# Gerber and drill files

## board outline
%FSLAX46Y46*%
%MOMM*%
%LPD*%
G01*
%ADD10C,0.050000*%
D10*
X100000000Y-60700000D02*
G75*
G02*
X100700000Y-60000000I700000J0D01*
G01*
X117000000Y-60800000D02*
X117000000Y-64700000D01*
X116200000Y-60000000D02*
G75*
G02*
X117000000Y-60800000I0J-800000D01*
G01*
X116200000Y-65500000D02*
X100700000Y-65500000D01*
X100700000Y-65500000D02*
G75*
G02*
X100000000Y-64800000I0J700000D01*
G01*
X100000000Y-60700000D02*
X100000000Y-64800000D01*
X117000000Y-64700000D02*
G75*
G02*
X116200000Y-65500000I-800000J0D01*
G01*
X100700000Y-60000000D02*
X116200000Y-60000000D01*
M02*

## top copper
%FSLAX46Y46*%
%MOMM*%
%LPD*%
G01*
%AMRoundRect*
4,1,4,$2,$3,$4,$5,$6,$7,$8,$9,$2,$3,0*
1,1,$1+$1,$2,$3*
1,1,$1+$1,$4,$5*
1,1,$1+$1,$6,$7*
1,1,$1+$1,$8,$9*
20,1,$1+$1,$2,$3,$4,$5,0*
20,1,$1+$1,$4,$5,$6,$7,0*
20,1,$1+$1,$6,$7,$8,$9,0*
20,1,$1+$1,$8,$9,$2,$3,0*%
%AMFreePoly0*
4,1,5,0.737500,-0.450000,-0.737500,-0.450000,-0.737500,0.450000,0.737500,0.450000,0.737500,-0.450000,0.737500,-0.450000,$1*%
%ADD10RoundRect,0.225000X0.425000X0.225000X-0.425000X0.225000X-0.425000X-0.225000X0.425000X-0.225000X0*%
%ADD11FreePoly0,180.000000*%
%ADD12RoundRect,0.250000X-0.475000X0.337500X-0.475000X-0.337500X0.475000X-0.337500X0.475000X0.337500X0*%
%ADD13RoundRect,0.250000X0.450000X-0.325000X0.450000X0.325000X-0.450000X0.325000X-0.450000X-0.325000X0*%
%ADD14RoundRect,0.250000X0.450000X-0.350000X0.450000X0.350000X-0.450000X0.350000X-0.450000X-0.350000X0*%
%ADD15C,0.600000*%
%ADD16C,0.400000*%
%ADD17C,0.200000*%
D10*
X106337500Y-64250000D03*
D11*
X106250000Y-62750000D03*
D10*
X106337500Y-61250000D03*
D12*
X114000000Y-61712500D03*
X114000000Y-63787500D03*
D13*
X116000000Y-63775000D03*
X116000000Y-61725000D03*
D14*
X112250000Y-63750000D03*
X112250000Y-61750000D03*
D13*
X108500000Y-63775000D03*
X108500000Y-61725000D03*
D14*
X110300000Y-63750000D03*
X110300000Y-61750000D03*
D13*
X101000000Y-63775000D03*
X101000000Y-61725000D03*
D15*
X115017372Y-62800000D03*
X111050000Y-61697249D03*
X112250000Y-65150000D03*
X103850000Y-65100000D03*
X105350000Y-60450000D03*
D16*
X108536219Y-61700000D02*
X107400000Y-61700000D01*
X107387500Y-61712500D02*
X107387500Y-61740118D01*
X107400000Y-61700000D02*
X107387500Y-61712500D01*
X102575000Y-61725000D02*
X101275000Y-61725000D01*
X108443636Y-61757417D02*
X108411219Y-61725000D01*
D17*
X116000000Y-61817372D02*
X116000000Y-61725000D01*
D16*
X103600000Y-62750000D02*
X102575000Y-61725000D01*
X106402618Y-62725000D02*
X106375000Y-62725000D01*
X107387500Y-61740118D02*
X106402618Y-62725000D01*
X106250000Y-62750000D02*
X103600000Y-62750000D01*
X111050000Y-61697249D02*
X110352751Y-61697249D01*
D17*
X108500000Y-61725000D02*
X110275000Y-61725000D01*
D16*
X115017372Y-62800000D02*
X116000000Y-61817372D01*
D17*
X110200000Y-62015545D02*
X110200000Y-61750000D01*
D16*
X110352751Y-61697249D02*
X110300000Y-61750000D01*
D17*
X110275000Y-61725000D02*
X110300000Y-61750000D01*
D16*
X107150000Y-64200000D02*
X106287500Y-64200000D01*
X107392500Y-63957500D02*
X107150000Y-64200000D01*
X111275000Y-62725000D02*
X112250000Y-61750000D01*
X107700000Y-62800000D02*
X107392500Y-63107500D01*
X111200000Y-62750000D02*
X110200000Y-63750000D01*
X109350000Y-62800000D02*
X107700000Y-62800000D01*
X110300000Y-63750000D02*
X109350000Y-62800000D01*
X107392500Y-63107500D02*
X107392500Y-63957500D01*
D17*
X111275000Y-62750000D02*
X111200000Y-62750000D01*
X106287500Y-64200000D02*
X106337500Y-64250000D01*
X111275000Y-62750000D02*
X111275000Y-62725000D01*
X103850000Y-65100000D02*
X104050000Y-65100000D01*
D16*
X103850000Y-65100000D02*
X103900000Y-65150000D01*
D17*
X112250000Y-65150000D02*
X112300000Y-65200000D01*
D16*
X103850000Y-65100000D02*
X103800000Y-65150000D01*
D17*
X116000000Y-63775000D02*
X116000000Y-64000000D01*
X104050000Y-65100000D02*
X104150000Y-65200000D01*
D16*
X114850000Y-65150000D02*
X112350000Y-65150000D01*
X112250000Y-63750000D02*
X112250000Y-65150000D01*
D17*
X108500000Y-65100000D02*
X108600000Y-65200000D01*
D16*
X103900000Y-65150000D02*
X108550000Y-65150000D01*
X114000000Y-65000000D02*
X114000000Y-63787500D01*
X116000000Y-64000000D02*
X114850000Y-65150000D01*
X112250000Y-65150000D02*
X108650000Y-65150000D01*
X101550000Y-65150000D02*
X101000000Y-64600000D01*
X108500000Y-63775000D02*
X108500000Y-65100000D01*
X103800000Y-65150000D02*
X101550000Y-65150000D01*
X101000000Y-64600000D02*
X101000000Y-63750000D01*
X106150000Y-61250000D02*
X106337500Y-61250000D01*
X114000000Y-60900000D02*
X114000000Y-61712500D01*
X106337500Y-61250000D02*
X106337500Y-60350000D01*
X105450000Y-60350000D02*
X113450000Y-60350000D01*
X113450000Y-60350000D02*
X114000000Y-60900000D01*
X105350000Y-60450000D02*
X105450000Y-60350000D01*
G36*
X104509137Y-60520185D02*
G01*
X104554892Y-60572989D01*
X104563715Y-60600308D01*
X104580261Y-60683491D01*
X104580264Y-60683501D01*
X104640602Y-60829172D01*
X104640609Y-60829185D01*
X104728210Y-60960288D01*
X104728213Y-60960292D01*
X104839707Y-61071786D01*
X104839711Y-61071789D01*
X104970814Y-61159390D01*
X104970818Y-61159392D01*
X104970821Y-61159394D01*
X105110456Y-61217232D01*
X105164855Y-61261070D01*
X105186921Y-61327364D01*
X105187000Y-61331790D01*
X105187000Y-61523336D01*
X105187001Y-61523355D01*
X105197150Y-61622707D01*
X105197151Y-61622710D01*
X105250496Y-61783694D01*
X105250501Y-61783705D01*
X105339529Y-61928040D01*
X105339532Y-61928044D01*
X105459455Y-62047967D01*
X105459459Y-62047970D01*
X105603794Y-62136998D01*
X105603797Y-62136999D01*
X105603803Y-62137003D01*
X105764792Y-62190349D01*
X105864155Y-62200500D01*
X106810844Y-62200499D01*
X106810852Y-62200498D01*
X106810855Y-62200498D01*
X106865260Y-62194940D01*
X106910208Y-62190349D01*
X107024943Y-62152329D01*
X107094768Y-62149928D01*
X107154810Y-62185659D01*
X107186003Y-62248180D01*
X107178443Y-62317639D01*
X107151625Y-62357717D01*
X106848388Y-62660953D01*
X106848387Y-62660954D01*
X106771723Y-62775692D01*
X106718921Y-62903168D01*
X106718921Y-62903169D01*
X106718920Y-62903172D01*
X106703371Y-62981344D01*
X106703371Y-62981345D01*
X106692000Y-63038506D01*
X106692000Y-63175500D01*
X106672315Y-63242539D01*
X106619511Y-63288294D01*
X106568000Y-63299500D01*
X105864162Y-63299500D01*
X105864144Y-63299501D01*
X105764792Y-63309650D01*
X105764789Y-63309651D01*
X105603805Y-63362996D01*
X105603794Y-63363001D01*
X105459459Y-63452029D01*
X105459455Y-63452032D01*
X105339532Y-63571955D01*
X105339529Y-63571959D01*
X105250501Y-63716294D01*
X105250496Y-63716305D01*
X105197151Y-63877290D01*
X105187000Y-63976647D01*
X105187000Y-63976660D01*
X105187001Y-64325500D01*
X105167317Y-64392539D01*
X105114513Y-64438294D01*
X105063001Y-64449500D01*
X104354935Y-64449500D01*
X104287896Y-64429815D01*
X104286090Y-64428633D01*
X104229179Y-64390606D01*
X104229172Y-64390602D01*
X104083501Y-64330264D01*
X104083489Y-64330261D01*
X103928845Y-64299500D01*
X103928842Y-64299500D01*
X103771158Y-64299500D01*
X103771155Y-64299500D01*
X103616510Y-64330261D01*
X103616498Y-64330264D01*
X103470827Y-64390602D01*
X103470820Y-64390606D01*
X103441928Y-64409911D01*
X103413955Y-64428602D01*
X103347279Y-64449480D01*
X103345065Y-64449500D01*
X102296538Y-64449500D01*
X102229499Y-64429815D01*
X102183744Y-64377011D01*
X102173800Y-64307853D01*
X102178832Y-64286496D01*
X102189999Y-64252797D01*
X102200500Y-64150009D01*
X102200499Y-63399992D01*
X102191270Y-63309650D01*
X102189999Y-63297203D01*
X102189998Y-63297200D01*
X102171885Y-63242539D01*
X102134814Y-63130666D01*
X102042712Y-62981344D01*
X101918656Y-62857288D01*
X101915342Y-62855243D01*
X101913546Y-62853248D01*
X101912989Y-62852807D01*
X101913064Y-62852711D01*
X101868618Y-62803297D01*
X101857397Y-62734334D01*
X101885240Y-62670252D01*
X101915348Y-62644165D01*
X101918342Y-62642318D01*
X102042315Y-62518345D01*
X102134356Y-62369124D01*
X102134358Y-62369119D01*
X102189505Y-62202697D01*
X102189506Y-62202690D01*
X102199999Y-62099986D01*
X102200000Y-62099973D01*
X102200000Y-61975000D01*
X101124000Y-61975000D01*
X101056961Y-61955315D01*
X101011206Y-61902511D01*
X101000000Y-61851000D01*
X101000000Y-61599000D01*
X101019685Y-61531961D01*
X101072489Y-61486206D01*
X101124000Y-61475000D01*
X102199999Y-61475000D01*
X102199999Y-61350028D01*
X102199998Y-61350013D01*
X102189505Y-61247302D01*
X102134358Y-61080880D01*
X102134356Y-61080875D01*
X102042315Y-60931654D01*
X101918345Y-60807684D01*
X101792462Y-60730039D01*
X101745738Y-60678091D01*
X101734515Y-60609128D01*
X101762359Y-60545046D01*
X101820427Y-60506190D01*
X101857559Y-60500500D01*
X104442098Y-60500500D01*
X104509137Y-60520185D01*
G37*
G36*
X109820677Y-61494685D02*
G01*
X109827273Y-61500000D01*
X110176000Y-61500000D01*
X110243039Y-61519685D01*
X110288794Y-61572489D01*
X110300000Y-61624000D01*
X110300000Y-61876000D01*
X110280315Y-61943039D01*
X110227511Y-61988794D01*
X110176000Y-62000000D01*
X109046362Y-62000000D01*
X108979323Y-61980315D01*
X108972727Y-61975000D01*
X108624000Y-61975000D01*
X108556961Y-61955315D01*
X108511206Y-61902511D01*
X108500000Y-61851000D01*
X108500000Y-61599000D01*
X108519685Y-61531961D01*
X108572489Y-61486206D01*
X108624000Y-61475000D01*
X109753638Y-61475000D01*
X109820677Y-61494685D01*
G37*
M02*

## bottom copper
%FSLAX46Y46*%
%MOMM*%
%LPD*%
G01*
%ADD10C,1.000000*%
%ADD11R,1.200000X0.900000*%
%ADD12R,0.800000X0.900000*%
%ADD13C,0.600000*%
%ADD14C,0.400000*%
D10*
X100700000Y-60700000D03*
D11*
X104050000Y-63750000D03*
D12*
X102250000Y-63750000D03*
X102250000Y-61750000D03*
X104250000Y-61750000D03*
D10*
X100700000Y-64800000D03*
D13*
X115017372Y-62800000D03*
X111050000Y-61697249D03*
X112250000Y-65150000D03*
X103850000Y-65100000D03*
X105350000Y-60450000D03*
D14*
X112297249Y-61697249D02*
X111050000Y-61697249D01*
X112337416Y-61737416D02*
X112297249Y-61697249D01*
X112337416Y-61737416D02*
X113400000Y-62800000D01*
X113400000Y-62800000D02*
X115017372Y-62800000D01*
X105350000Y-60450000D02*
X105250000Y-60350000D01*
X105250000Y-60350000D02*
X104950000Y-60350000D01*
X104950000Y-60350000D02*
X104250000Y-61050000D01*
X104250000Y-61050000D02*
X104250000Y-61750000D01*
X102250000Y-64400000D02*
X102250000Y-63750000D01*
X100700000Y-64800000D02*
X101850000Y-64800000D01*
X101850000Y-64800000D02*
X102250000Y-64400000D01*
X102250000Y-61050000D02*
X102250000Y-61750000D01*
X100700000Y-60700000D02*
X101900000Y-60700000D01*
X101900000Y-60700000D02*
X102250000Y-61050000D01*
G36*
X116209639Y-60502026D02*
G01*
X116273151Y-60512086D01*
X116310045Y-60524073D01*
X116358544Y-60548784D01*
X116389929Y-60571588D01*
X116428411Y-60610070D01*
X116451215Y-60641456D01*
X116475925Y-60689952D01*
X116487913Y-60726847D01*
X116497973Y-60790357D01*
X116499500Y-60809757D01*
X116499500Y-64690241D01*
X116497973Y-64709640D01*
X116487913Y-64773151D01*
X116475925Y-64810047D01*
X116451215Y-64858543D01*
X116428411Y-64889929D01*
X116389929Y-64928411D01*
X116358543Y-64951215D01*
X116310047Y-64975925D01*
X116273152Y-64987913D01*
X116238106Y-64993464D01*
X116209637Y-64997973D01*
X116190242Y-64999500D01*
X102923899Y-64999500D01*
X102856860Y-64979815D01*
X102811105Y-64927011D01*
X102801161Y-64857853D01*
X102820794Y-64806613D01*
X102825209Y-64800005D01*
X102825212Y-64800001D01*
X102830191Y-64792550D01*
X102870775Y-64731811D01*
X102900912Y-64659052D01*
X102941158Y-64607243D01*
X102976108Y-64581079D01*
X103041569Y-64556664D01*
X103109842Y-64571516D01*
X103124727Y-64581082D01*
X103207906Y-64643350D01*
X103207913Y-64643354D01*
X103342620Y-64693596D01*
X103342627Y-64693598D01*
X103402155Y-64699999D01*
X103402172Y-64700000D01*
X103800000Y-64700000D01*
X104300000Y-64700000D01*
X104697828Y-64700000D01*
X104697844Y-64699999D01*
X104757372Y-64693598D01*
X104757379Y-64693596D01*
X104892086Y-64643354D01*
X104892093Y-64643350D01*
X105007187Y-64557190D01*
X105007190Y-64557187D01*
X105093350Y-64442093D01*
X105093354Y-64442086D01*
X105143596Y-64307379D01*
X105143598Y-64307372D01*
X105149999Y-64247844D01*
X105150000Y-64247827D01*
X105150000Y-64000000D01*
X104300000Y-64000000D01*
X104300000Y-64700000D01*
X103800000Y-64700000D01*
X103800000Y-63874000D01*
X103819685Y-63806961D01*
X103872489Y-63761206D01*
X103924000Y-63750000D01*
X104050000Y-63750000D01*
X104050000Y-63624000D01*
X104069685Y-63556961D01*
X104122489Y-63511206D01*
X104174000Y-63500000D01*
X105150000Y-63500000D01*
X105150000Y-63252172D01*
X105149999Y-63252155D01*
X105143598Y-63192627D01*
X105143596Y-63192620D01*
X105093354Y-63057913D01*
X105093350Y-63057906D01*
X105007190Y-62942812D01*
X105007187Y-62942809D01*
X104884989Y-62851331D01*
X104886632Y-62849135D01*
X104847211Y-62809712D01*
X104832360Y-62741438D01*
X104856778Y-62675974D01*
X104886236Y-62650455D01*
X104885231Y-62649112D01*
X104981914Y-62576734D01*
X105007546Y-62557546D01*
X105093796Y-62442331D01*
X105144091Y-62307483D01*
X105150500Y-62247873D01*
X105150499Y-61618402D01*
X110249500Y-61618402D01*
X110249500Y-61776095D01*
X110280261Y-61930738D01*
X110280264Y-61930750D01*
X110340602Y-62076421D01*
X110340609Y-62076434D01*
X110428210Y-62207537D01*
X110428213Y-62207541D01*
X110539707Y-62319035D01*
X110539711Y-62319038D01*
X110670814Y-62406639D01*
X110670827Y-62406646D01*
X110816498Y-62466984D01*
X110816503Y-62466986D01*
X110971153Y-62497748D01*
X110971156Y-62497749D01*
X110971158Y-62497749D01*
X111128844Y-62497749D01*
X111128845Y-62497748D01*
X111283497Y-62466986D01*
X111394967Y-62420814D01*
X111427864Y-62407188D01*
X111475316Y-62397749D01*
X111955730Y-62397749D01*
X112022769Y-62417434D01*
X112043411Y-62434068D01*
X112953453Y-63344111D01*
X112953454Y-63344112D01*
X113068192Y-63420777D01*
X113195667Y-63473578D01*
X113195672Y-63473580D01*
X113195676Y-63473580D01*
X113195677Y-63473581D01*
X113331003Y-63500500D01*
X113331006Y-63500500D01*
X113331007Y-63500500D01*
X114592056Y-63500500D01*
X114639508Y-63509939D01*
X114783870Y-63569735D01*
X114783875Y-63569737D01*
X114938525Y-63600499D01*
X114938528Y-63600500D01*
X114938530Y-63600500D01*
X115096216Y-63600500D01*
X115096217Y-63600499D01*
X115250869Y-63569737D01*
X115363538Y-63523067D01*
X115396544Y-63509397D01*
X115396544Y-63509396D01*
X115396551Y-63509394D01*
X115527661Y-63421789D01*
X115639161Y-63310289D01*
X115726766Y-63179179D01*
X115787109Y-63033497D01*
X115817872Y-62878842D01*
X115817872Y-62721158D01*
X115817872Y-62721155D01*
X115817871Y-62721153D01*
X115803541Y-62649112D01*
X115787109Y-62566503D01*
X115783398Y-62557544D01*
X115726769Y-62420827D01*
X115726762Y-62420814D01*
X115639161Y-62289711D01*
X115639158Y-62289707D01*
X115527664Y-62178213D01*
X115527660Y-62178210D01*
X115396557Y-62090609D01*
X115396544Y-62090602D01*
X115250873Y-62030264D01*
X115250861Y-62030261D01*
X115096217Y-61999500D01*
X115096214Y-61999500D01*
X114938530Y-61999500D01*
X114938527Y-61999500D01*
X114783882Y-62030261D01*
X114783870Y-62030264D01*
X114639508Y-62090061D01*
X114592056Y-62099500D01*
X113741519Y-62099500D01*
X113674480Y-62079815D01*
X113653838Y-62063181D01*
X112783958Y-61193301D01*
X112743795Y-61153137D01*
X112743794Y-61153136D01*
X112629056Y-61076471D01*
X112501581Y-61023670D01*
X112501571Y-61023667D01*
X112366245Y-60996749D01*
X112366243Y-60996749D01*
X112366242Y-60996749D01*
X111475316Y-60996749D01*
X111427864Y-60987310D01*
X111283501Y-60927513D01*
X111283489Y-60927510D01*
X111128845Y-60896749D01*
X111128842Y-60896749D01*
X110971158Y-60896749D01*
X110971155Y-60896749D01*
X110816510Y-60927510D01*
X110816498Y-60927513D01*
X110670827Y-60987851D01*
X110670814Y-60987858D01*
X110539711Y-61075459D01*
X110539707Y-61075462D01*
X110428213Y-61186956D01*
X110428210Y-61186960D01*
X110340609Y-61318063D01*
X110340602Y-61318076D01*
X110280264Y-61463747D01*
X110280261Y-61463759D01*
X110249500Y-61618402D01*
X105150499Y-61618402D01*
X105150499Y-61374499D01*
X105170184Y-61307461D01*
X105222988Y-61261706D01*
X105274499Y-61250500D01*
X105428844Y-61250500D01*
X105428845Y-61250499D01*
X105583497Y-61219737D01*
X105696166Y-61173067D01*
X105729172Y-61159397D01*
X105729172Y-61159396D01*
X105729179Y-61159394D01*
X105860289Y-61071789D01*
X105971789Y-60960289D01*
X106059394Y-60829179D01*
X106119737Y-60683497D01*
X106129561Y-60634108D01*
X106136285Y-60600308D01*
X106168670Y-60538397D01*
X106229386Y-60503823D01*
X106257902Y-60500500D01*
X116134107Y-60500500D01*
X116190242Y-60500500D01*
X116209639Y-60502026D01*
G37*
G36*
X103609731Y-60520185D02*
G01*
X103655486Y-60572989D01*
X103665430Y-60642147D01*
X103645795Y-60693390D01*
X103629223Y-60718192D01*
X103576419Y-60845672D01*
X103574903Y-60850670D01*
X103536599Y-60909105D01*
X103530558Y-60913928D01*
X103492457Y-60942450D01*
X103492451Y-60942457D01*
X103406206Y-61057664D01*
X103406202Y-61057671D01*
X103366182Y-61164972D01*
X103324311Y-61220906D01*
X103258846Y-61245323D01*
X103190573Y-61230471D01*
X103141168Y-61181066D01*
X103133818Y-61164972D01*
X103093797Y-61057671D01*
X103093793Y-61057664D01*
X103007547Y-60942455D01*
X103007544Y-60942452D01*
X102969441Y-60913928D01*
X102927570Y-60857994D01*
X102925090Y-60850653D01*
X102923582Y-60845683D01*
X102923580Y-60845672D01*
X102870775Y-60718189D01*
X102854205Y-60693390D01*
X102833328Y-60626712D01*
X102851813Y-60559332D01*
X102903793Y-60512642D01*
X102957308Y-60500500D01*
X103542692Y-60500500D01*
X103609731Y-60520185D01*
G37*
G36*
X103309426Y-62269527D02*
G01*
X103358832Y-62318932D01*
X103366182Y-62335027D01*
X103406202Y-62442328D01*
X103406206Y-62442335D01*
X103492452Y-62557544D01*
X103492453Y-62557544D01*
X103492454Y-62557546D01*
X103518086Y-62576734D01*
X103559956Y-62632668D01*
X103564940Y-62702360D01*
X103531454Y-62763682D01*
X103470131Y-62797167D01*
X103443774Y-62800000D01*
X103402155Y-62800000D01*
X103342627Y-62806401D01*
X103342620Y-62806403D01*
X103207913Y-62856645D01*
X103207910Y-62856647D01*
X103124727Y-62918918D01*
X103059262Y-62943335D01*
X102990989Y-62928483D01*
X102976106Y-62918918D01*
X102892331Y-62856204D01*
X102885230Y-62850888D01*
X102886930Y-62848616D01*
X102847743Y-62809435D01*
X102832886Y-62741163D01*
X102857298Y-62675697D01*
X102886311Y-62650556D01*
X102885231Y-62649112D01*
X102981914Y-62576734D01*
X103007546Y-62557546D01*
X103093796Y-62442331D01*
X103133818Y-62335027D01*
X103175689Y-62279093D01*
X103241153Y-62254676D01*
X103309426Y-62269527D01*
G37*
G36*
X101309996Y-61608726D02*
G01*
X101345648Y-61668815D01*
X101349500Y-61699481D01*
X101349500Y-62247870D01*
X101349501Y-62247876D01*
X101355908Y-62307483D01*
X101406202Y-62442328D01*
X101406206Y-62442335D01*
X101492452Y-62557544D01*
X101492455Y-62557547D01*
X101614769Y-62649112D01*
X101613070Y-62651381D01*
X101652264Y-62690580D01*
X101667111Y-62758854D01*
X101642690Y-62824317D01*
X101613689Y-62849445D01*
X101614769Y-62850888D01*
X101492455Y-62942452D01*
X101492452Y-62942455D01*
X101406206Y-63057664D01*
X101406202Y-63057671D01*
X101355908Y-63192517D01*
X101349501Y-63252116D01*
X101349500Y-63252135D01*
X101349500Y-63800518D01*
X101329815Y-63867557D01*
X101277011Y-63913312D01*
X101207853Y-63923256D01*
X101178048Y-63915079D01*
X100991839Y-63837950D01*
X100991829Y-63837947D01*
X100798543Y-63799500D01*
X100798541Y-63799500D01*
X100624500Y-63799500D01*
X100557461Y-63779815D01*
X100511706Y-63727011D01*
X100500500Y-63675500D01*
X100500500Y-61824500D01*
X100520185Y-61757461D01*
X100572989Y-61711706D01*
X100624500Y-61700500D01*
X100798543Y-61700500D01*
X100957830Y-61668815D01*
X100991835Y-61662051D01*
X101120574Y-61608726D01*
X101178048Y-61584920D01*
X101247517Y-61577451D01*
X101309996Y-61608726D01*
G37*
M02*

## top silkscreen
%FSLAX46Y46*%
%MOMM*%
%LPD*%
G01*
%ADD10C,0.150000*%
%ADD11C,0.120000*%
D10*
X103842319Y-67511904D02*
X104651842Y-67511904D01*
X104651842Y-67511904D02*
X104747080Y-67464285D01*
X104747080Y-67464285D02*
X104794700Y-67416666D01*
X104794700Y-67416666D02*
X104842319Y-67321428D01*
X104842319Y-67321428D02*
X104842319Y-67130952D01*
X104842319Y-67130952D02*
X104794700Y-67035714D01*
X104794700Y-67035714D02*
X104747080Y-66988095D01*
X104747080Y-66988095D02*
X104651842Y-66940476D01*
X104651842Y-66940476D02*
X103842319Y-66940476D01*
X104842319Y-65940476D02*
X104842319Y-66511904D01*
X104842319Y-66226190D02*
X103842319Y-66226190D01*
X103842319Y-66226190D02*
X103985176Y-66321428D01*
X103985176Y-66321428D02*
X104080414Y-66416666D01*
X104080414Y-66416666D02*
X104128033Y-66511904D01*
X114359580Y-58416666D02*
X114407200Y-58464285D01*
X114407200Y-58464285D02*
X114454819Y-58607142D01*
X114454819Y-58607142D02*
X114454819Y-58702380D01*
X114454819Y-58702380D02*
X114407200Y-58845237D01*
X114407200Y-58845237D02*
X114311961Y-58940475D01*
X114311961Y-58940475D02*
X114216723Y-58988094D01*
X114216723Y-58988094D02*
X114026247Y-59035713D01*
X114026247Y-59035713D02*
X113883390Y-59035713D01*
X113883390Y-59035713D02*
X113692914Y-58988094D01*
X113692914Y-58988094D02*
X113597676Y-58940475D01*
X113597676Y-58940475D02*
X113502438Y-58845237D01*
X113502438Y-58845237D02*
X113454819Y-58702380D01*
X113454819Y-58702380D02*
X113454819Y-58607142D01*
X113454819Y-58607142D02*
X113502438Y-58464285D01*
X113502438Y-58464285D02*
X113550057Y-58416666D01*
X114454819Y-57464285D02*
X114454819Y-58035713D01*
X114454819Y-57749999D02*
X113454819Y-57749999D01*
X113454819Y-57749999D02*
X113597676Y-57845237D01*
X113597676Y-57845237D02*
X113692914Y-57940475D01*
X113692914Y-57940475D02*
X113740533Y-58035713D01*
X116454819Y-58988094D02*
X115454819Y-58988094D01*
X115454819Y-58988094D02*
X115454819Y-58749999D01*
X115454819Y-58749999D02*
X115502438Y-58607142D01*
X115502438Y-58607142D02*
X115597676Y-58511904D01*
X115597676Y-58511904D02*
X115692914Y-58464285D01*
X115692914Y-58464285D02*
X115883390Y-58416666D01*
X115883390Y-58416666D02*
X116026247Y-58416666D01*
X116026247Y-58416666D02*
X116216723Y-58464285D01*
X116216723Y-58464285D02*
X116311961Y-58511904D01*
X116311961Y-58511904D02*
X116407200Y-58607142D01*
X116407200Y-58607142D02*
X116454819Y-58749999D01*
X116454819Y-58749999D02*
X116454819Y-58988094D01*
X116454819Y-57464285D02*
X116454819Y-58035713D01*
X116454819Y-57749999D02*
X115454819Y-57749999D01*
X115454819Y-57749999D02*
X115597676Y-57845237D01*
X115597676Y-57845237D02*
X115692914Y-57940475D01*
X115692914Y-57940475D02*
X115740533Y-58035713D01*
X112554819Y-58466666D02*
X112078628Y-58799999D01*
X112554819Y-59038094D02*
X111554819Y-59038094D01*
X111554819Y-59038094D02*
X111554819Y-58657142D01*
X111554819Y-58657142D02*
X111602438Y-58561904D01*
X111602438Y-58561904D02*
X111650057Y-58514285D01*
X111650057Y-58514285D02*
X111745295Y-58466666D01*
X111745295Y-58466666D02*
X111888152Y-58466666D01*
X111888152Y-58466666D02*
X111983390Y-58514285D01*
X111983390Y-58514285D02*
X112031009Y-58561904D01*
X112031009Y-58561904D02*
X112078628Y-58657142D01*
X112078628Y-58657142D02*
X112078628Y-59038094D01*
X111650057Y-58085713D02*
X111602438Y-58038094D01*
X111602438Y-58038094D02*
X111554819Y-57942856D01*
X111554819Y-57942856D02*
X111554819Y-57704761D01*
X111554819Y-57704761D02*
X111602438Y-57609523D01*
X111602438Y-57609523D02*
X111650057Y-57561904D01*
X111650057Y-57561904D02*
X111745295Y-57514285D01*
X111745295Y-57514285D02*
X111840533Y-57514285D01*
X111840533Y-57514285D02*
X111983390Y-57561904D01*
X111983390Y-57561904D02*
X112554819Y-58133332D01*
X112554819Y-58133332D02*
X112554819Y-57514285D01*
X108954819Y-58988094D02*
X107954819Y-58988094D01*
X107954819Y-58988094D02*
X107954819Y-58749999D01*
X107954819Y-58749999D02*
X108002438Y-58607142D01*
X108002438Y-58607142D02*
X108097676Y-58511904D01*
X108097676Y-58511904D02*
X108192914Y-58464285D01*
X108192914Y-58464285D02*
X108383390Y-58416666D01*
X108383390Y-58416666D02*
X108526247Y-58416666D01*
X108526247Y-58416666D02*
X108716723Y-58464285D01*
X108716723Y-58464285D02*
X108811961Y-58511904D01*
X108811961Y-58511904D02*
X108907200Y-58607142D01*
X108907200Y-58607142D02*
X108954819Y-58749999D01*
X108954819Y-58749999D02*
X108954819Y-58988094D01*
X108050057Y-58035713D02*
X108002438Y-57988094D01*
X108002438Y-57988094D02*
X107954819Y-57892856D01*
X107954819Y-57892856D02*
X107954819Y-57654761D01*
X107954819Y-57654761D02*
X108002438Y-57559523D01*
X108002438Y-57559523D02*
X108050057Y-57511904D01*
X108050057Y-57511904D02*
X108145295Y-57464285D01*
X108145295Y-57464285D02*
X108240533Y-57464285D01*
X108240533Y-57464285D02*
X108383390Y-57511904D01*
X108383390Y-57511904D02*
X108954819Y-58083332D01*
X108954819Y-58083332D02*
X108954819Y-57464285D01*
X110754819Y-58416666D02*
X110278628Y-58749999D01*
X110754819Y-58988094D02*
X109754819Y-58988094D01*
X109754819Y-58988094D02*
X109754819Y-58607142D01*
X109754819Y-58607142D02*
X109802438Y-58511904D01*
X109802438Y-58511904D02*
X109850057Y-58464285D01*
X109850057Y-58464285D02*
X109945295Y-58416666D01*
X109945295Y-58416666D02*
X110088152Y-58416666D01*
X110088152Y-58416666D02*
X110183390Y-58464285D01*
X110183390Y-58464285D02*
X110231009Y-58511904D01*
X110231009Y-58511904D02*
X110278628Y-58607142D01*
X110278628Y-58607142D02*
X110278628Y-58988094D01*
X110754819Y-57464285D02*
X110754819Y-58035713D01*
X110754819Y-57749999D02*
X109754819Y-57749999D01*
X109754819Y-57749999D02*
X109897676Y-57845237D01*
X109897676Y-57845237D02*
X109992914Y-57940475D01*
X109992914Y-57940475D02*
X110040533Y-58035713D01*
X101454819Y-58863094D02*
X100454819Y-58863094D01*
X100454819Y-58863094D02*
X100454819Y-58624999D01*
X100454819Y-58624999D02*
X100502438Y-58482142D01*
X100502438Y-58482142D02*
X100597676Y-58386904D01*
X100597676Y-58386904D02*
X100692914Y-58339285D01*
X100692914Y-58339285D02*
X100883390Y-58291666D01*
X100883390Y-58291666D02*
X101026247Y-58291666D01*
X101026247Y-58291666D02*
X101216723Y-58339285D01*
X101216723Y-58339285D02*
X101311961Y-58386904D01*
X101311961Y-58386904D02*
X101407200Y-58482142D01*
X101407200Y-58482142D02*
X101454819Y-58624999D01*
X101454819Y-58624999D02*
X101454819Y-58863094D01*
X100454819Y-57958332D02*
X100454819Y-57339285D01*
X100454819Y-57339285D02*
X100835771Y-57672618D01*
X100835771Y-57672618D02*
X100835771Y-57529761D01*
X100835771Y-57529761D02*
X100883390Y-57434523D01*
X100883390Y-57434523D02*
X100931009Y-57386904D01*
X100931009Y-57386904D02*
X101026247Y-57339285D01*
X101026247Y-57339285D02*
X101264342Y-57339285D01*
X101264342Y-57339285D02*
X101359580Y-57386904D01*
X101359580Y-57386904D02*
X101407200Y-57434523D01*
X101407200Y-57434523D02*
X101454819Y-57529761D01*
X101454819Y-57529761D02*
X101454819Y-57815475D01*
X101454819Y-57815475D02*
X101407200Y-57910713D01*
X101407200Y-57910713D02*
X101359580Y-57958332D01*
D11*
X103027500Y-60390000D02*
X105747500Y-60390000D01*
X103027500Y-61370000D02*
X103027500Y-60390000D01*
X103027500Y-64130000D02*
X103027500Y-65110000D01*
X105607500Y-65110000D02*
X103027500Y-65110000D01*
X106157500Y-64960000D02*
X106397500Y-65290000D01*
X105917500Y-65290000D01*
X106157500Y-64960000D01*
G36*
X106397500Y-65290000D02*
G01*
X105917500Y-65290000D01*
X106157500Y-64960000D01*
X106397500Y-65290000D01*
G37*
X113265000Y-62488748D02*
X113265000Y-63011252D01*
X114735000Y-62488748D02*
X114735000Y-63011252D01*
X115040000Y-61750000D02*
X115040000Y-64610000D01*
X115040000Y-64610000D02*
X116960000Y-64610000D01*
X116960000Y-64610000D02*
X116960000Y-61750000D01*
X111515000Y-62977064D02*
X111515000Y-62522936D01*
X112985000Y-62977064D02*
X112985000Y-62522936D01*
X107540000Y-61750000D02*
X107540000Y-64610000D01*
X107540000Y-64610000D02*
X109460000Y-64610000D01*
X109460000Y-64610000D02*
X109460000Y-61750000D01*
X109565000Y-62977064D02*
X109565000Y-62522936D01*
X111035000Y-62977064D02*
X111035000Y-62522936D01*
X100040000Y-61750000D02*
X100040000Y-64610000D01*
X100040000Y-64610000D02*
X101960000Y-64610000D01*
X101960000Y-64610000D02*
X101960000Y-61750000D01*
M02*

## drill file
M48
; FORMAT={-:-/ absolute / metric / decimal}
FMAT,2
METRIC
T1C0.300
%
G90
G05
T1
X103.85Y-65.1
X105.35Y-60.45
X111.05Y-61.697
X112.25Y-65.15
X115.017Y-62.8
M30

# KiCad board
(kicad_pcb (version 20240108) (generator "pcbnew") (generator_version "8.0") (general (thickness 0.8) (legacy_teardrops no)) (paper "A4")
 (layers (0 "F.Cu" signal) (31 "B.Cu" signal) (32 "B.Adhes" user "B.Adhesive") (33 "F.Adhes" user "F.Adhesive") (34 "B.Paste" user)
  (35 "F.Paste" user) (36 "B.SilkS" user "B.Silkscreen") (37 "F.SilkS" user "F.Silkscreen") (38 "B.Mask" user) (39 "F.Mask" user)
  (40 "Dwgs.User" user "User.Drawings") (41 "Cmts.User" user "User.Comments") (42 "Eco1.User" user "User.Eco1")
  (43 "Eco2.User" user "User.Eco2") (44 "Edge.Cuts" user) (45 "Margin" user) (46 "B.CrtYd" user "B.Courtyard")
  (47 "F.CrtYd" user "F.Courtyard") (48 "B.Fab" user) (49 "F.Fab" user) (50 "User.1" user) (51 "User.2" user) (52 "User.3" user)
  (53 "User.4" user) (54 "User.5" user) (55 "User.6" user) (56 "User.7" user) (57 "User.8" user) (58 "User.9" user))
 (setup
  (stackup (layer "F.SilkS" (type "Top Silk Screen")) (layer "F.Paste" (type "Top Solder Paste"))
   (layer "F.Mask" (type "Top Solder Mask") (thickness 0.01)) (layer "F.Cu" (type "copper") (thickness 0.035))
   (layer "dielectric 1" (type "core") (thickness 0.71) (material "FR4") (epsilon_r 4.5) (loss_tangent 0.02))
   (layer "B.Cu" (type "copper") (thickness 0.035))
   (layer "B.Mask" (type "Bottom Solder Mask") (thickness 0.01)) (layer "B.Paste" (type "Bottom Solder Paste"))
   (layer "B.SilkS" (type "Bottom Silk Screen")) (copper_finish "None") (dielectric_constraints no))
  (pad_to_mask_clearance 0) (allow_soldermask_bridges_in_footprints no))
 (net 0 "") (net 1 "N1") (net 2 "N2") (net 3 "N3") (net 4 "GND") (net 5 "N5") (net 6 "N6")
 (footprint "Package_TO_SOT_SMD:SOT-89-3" (layer "F.Cu") (at 104.3875 62.75 180)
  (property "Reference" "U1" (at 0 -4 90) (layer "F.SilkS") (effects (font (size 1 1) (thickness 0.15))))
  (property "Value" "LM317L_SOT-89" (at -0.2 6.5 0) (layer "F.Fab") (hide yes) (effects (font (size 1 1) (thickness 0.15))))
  (fp_line (start 1.36 2.36) (end -1.36 2.36) (stroke (width 0.12) (type solid)) (layer "F.SilkS"))
  (fp_line (start 1.36 1.38) (end 1.36 2.36) (stroke (width 0.12) (type solid)) (layer "F.SilkS"))
  (fp_line (start 1.36 -1.38) (end 1.36 -2.36) (stroke (width 0.12) (type solid)) (layer "F.SilkS"))
  (fp_line (start -1.22 -2.36) (end 1.36 -2.36) (stroke (width 0.12) (type solid)) (layer "F.SilkS"))
  (fp_poly
   (pts (xy -1.77 -2.21) (xy -2.01 -2.54) (xy -1.53 -2.54) (xy -1.77 -2.21)) (stroke (width 0.12) (type solid)) (fill solid)
   (layer "F.SilkS"))
  (pad "1" smd roundrect (at -1.95 -1.5 180) (size 1.3 0.9) (layers "F.Cu" "F.Paste" "F.Mask") (roundrect_rratio 0.25) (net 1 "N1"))
  (pad "2" smd custom (at -1.8625 0 180) (size 1.475 0.9) (layers "F.Cu" "F.Paste" "F.Mask") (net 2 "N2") (zone_connect 2)
   (thermal_bridge_angle 45) (options (clearance outline) (anchor rect)) (primitives))
  (pad "3" smd roundrect (at -1.95 1.5 180) (size 1.3 0.9) (layers "F.Cu" "F.Paste" "F.Mask") (roundrect_rratio 0.25) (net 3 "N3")))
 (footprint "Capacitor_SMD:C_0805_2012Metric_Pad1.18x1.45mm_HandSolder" (layer "F.Cu") (at 114 62.75 -90)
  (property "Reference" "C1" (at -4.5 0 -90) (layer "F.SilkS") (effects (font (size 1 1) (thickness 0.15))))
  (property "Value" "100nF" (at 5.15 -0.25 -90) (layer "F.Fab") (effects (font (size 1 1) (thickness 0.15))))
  (fp_line (start -0.261252 0.735) (end 0.261252 0.735) (stroke (width 0.12) (type solid)) (layer "F.SilkS"))
  (fp_line (start -0.261252 -0.735) (end 0.261252 -0.735) (stroke (width 0.12) (type solid)) (layer "F.SilkS"))
  (pad "1" smd roundrect (at -1.0375 0 270) (size 1.175 1.45) (layers "F.Cu" "F.Paste" "F.Mask") (roundrect_rratio 0.212766) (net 3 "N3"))
  (pad "2" smd roundrect (at 1.0375 0 270) (size 1.175 1.45) (layers "F.Cu" "F.Paste" "F.Mask") (roundrect_rratio 0.212766) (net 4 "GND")))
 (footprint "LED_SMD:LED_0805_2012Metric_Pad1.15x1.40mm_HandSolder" (layer "F.Cu") (at 116 62.75 90)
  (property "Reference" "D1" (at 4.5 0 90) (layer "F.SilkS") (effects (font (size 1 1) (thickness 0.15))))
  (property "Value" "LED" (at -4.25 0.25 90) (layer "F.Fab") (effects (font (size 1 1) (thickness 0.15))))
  (fp_line (start 1 -0.96) (end -1.86 -0.96) (stroke (width 0.12) (type solid)) (layer "F.SilkS"))
  (fp_line (start -1.86 -0.96) (end -1.86 0.96) (stroke (width 0.12) (type solid)) (layer "F.SilkS"))
  (fp_line (start -1.86 0.96) (end 1 0.96) (stroke (width 0.12) (type solid)) (layer "F.SilkS"))
  (pad "1" smd roundrect (at -1.025 0 90) (size 1.15 1.4) (layers "F.Cu" "F.Paste" "F.Mask") (roundrect_rratio 0.217391) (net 4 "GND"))
  (pad "2" smd roundrect (at 1.025 0 90) (size 1.15 1.4) (layers "F.Cu" "F.Paste" "F.Mask") (roundrect_rratio 0.217391) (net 2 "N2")))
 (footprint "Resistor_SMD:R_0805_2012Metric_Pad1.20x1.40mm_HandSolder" (layer "F.Cu") (at 112.25 62.75 90)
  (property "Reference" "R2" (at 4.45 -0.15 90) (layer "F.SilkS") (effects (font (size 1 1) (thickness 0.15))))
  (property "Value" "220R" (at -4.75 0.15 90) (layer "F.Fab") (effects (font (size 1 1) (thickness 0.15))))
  (fp_line (start -0.227064 -0.735) (end 0.227064 -0.735) (stroke (width 0.12) (type solid)) (layer "F.SilkS"))
  (fp_line (start -0.227064 0.735) (end 0.227064 0.735) (stroke (width 0.12) (type solid)) (layer "F.SilkS"))
  (pad "1" smd roundrect (at -1 0 90) (size 1.2 1.4) (layers "F.Cu" "F.Paste" "F.Mask") (roundrect_rratio 0.208333) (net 4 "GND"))
  (pad "2" smd roundrect (at 1 0 90) (size 1.2 1.4) (layers "F.Cu" "F.Paste" "F.Mask") (roundrect_rratio 0.208333) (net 1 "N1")))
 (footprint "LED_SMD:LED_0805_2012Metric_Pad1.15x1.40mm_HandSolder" (layer "F.Cu") (at 108.5 62.75 90)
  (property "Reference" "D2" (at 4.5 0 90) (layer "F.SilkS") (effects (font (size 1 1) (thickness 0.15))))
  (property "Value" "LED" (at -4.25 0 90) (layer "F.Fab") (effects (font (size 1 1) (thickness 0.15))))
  (fp_line (start 1 -0.96) (end -1.86 -0.96) (stroke (width 0.12) (type solid)) (layer "F.SilkS"))
  (fp_line (start -1.86 -0.96) (end -1.86 0.96) (stroke (width 0.12) (type solid)) (layer "F.SilkS"))
  (fp_line (start -1.86 0.96) (end 1 0.96) (stroke (width 0.12) (type solid)) (layer "F.SilkS"))
  (pad "1" smd roundrect (at -1.025 0 90) (size 1.15 1.4) (layers "F.Cu" "F.Paste" "F.Mask") (roundrect_rratio 0.217391) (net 4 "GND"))
  (pad "2" smd roundrect (at 1.025 0 90) (size 1.15 1.4) (layers "F.Cu" "F.Paste" "F.Mask") (roundrect_rratio 0.217391) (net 2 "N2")))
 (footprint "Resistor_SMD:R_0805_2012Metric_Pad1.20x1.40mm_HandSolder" (layer "F.Cu") (at 110.3 62.75 90)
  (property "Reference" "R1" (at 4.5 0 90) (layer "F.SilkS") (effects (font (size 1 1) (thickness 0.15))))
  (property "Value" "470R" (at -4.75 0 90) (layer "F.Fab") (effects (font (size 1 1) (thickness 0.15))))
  (fp_line (start -0.227064 -0.735) (end 0.227064 -0.735) (stroke (width 0.12) (type solid)) (layer "F.SilkS"))
  (fp_line (start -0.227064 0.735) (end 0.227064 0.735) (stroke (width 0.12) (type solid)) (layer "F.SilkS"))
  (pad "1" smd roundrect (at -1 0 90) (size 1.2 1.4) (layers "F.Cu" "F.Paste" "F.Mask") (roundrect_rratio 0.208333) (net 1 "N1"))
  (pad "2" smd roundrect (at 1 0 90) (size 1.2 1.4) (layers "F.Cu" "F.Paste" "F.Mask") (roundrect_rratio 0.208333) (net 2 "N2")))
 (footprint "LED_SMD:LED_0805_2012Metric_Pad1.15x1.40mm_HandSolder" (layer "F.Cu") (at 101 62.75 90)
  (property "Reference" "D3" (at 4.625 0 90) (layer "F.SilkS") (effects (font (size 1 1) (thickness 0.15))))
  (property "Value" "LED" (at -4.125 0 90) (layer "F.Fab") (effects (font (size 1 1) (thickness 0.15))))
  (fp_line (start 1 -0.96) (end -1.86 -0.96) (stroke (width 0.12) (type solid)) (layer "F.SilkS"))
  (fp_line (start -1.86 -0.96) (end -1.86 0.96) (stroke (width 0.12) (type solid)) (layer "F.SilkS"))
  (fp_line (start -1.86 0.96) (end 1 0.96) (stroke (width 0.12) (type solid)) (layer "F.SilkS"))
  (pad "1" smd roundrect (at -1.025 0 90) (size 1.15 1.4) (layers "F.Cu" "F.Paste" "F.Mask") (roundrect_rratio 0.217391) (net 4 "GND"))
  (pad "2" smd roundrect (at 1.025 0 90) (size 1.15 1.4) (layers "F.Cu" "F.Paste" "F.Mask") (roundrect_rratio 0.217391) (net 2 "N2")))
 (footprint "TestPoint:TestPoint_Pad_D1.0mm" (layer "B.Cu") (at 100.7 60.7 180)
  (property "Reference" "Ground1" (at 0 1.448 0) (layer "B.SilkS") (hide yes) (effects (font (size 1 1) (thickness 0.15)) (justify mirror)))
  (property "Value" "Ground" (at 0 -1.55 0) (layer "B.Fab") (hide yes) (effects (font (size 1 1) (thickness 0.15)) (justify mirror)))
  (pad "1" smd circle (at 0 0 180) (size 1 1) (layers "B.Cu" "B.Mask") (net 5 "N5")))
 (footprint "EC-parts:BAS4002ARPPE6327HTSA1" (layer "B.Cu") (at 103.25 62.75 180)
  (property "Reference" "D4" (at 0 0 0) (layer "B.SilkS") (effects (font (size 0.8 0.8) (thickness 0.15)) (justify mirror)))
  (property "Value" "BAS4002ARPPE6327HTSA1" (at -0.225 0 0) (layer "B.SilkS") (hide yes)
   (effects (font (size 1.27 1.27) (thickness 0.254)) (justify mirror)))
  (pad "1" smd rect (at -0.8 -1 90) (size 0.9 1.2) (layers "B.Cu" "B.Paste" "B.Mask") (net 4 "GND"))
  (pad "2" smd rect (at 1 -1 180) (size 0.8 0.9) (layers "B.Cu" "B.Paste" "B.Mask") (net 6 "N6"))
  (pad "3" smd rect (at 1 1 180) (size 0.8 0.9) (layers "B.Cu" "B.Paste" "B.Mask") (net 5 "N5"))
  (pad "4" smd rect (at -1 1 180) (size 0.8 0.9) (layers "B.Cu" "B.Paste" "B.Mask") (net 3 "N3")))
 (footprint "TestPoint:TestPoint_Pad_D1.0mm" (layer "B.Cu") (at 100.7 64.8 180)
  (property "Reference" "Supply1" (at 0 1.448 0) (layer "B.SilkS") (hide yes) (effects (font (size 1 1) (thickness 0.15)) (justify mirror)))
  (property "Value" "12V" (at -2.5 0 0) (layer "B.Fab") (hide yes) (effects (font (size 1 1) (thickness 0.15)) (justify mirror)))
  (pad "1" smd circle (at 0 0 180) (size 1 1) (layers "B.Cu" "B.Mask") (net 6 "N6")))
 (gr_arc (start 100 60.7) (mid 100.205025 60.205025) (end 100.7 60) (stroke (width 0.05) (type default)) (layer "Edge.Cuts"))
 (gr_line (start 117 60.8) (end 117 64.7) (stroke (width 0.05) (type default)) (layer "Edge.Cuts"))
 (gr_arc (start 116.2 60) (mid 116.765685 60.234315) (end 117 60.8) (stroke (width 0.05) (type default)) (layer "Edge.Cuts"))
 (gr_line (start 116.2 65.5) (end 100.7 65.5) (stroke (width 0.05) (type default)) (layer "Edge.Cuts"))
 (gr_arc (start 100.7 65.5) (mid 100.205025 65.294975) (end 100 64.8) (stroke (width 0.05) (type default)) (layer "Edge.Cuts"))
 (gr_line (start 100 60.7) (end 100 64.8) (stroke (width 0.05) (type default)) (layer "Edge.Cuts"))
 (gr_arc (start 117 64.7) (mid 116.765685 65.265685) (end 116.2 65.5) (stroke (width 0.05) (type default)) (layer "Edge.Cuts"))
 (gr_line (start 100.7 60) (end 116.2 60) (stroke (width 0.05) (type default)) (layer "Edge.Cuts"))
 (segment (start 108.536219 61.7) (end 107.4 61.7) (width 0.4) (layer "F.Cu") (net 2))
 (segment (start 107.3875 61.7125) (end 107.3875 61.740118) (width 0.4) (layer "F.Cu") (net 2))
 (segment (start 107.4 61.7) (end 107.3875 61.7125) (width 0.4) (layer "F.Cu") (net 2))
 (segment (start 102.575 61.725) (end 101.275 61.725) (width 0.4) (layer "F.Cu") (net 2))
 (segment (start 108.443636 61.757417) (end 108.411219 61.725) (width 0.4) (layer "F.Cu") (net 2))
 (segment (start 116 61.817372) (end 116 61.725) (width 0.2) (layer "F.Cu") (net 2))
 (segment (start 103.6 62.75) (end 102.575 61.725) (width 0.4) (layer "F.Cu") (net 2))
 (segment (start 106.402618 62.725) (end 106.375 62.725) (width 0.4) (layer "F.Cu") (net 2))
 (segment (start 107.3875 61.740118) (end 106.402618 62.725) (width 0.4) (layer "F.Cu") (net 2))
 (segment (start 106.25 62.75) (end 103.6 62.75) (width 0.4) (layer "F.Cu") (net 2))
 (segment (start 111.05 61.697249) (end 110.352751 61.697249) (width 0.4) (layer "F.Cu") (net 2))
 (segment (start 108.5 61.725) (end 110.275 61.725) (width 0.2) (layer "F.Cu") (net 2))
 (segment (start 115.017372 62.8) (end 116 61.817372) (width 0.4) (layer "F.Cu") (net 2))
 (segment (start 110.2 62.015545) (end 110.2 61.75) (width 0.2) (layer "F.Cu") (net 2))
 (segment (start 110.352751 61.697249) (end 110.3 61.75) (width 0.4) (layer "F.Cu") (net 2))
 (segment (start 110.275 61.725) (end 110.3 61.75) (width 0.2) (layer "F.Cu") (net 2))
 (via (at 115.017372 62.8) (size 0.6) (drill 0.3) (layers "F.Cu" "B.Cu") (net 2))
 (via (at 111.05 61.697249) (size 0.6) (drill 0.3) (layers "F.Cu" "B.Cu") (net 2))
 (segment (start 112.297249 61.697249) (end 111.05 61.697249) (width 0.4) (layer "B.Cu") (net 2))
 (segment (start 112.337416 61.737416) (end 112.297249 61.697249) (width 0.4) (layer "B.Cu") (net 2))
 (segment (start 112.337416 61.737416) (end 113.4 62.8) (width 0.4) (layer "B.Cu") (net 2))
 (segment (start 113.4 62.8) (end 115.017372 62.8) (width 0.4) (layer "B.Cu") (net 2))
 (segment (start 107.15 64.2) (end 106.2875 64.2) (width 0.4) (layer "F.Cu") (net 1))
 (segment (start 107.3925 63.9575) (end 107.15 64.2) (width 0.4) (layer "F.Cu") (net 1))
 (segment (start 111.275 62.725) (end 112.25 61.75) (width 0.4) (layer "F.Cu") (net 1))
 (segment (start 107.7 62.8) (end 107.3925 63.1075) (width 0.4) (layer "F.Cu") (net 1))
 (segment (start 111.2 62.75) (end 110.2 63.75) (width 0.4) (layer "F.Cu") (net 1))
 (segment (start 109.35 62.8) (end 107.7 62.8) (width 0.4) (layer "F.Cu") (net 1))
 (segment (start 110.3 63.75) (end 109.35 62.8) (width 0.4) (layer "F.Cu") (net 1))
 (segment (start 107.3925 63.1075) (end 107.3925 63.9575) (width 0.4) (layer "F.Cu") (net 1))
 (segment (start 111.275 62.75) (end 111.2 62.75) (width 0.2) (layer "F.Cu") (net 1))
 (segment (start 106.2875 64.2) (end 106.3375 64.25) (width 0.2) (layer "F.Cu") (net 1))
 (segment (start 111.275 62.75) (end 111.275 62.725) (width 0.2) (layer "F.Cu") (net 1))
 (segment (start 103.85 65.1) (end 104.05 65.1) (width 0.2) (layer "F.Cu") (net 4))
 (segment (start 103.85 65.1) (end 103.9 65.15) (width 0.4) (layer "F.Cu") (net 4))
 (segment (start 112.25 65.15) (end 112.3 65.2) (width 0.2) (layer "F.Cu") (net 4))
 (segment (start 103.85 65.1) (end 103.8 65.15) (width 0.4) (layer "F.Cu") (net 4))
 (segment (start 116 63.775) (end 116 64) (width 0.2) (layer "F.Cu") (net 4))
 (segment (start 104.05 65.1) (end 104.15 65.2) (width 0.2) (layer "F.Cu") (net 4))
 (segment (start 114.85 65.15) (end 112.35 65.15) (width 0.4) (layer "F.Cu") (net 4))
 (segment (start 112.25 63.75) (end 112.25 65.15) (width 0.4) (layer "F.Cu") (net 4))
 (segment (start 108.5 65.1) (end 108.6 65.2) (width 0.2) (layer "F.Cu") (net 4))
 (segment (start 103.9 65.15) (end 108.55 65.15) (width 0.4) (layer "F.Cu") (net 4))
 (segment (start 114 65) (end 114 63.7875) (width 0.4) (layer "F.Cu") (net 4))
 (segment (start 116 64) (end 114.85 65.15) (width 0.4) (layer "F.Cu") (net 4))
 (segment (start 112.25 65.15) (end 108.65 65.15) (width 0.4) (layer "F.Cu") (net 4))
 (segment (start 101.55 65.15) (end 101 64.6) (width 0.4) (layer "F.Cu") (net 4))
 (segment (start 108.5 63.775) (end 108.5 65.1) (width 0.4) (layer "F.Cu") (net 4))
 (segment (start 103.8 65.15) (end 101.55 65.15) (width 0.4) (layer "F.Cu") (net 4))
 (segment (start 101 64.6) (end 101 63.75) (width 0.4) (layer "F.Cu") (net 4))
 (via (at 112.25 65.15) (size 0.6) (drill 0.3) (layers "F.Cu" "B.Cu") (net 4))
 (via (at 103.85 65.1) (size 0.6) (drill 0.3) (layers "F.Cu" "B.Cu") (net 4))
 (segment (start 106.15 61.25) (end 106.3375 61.25) (width 0.4) (layer "F.Cu") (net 3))
 (segment (start 114 60.9) (end 114 61.7125) (width 0.4) (layer "F.Cu") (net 3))
 (segment (start 106.3375 61.25) (end 106.3375 60.35) (width 0.4) (layer "F.Cu") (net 3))
 (segment (start 105.45 60.35) (end 113.45 60.35) (width 0.4) (layer "F.Cu") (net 3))
 (segment (start 113.45 60.35) (end 114 60.9) (width 0.4) (layer "F.Cu") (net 3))
 (segment (start 105.35 60.45) (end 105.45 60.35) (width 0.4) (layer "F.Cu") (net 3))
 (via (at 105.35 60.45) (size 0.6) (drill 0.3) (layers "F.Cu" "B.Cu") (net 3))
 (segment (start 105.35 60.45) (end 105.25 60.35) (width 0.4) (layer "B.Cu") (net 3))
 (segment (start 105.25 60.35) (end 104.95 60.35) (width 0.4) (layer "B.Cu") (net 3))
 (segment (start 104.95 60.35) (end 104.25 61.05) (width 0.4) (layer "B.Cu") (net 3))
 (segment (start 104.25 61.05) (end 104.25 61.75) (width 0.4) (layer "B.Cu") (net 3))
 (segment (start 102.25 64.4) (end 102.25 63.75) (width 0.4) (layer "B.Cu") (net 6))
 (segment (start 100.7 64.8) (end 101.85 64.8) (width 0.4) (layer "B.Cu") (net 6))
 (segment (start 101.85 64.8) (end 102.25 64.4) (width 0.4) (layer "B.Cu") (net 6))
 (segment (start 102.25 61.05) (end 102.25 61.75) (width 0.4) (layer "B.Cu") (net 5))
 (segment (start 100.7 60.7) (end 101.9 60.7) (width 0.4) (layer "B.Cu") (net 5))
 (segment (start 101.9 60.7) (end 102.25 61.05) (width 0.4) (layer "B.Cu") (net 5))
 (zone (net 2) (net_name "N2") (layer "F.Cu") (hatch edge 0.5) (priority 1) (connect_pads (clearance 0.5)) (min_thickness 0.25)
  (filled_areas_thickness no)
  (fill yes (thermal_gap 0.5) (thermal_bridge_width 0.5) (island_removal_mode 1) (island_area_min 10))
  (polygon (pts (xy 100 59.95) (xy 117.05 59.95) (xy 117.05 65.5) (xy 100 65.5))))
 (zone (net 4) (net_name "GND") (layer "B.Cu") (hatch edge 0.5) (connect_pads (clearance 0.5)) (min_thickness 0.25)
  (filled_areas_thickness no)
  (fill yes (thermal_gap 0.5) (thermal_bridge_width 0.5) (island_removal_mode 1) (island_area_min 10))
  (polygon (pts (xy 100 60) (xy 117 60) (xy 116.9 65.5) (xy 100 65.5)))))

